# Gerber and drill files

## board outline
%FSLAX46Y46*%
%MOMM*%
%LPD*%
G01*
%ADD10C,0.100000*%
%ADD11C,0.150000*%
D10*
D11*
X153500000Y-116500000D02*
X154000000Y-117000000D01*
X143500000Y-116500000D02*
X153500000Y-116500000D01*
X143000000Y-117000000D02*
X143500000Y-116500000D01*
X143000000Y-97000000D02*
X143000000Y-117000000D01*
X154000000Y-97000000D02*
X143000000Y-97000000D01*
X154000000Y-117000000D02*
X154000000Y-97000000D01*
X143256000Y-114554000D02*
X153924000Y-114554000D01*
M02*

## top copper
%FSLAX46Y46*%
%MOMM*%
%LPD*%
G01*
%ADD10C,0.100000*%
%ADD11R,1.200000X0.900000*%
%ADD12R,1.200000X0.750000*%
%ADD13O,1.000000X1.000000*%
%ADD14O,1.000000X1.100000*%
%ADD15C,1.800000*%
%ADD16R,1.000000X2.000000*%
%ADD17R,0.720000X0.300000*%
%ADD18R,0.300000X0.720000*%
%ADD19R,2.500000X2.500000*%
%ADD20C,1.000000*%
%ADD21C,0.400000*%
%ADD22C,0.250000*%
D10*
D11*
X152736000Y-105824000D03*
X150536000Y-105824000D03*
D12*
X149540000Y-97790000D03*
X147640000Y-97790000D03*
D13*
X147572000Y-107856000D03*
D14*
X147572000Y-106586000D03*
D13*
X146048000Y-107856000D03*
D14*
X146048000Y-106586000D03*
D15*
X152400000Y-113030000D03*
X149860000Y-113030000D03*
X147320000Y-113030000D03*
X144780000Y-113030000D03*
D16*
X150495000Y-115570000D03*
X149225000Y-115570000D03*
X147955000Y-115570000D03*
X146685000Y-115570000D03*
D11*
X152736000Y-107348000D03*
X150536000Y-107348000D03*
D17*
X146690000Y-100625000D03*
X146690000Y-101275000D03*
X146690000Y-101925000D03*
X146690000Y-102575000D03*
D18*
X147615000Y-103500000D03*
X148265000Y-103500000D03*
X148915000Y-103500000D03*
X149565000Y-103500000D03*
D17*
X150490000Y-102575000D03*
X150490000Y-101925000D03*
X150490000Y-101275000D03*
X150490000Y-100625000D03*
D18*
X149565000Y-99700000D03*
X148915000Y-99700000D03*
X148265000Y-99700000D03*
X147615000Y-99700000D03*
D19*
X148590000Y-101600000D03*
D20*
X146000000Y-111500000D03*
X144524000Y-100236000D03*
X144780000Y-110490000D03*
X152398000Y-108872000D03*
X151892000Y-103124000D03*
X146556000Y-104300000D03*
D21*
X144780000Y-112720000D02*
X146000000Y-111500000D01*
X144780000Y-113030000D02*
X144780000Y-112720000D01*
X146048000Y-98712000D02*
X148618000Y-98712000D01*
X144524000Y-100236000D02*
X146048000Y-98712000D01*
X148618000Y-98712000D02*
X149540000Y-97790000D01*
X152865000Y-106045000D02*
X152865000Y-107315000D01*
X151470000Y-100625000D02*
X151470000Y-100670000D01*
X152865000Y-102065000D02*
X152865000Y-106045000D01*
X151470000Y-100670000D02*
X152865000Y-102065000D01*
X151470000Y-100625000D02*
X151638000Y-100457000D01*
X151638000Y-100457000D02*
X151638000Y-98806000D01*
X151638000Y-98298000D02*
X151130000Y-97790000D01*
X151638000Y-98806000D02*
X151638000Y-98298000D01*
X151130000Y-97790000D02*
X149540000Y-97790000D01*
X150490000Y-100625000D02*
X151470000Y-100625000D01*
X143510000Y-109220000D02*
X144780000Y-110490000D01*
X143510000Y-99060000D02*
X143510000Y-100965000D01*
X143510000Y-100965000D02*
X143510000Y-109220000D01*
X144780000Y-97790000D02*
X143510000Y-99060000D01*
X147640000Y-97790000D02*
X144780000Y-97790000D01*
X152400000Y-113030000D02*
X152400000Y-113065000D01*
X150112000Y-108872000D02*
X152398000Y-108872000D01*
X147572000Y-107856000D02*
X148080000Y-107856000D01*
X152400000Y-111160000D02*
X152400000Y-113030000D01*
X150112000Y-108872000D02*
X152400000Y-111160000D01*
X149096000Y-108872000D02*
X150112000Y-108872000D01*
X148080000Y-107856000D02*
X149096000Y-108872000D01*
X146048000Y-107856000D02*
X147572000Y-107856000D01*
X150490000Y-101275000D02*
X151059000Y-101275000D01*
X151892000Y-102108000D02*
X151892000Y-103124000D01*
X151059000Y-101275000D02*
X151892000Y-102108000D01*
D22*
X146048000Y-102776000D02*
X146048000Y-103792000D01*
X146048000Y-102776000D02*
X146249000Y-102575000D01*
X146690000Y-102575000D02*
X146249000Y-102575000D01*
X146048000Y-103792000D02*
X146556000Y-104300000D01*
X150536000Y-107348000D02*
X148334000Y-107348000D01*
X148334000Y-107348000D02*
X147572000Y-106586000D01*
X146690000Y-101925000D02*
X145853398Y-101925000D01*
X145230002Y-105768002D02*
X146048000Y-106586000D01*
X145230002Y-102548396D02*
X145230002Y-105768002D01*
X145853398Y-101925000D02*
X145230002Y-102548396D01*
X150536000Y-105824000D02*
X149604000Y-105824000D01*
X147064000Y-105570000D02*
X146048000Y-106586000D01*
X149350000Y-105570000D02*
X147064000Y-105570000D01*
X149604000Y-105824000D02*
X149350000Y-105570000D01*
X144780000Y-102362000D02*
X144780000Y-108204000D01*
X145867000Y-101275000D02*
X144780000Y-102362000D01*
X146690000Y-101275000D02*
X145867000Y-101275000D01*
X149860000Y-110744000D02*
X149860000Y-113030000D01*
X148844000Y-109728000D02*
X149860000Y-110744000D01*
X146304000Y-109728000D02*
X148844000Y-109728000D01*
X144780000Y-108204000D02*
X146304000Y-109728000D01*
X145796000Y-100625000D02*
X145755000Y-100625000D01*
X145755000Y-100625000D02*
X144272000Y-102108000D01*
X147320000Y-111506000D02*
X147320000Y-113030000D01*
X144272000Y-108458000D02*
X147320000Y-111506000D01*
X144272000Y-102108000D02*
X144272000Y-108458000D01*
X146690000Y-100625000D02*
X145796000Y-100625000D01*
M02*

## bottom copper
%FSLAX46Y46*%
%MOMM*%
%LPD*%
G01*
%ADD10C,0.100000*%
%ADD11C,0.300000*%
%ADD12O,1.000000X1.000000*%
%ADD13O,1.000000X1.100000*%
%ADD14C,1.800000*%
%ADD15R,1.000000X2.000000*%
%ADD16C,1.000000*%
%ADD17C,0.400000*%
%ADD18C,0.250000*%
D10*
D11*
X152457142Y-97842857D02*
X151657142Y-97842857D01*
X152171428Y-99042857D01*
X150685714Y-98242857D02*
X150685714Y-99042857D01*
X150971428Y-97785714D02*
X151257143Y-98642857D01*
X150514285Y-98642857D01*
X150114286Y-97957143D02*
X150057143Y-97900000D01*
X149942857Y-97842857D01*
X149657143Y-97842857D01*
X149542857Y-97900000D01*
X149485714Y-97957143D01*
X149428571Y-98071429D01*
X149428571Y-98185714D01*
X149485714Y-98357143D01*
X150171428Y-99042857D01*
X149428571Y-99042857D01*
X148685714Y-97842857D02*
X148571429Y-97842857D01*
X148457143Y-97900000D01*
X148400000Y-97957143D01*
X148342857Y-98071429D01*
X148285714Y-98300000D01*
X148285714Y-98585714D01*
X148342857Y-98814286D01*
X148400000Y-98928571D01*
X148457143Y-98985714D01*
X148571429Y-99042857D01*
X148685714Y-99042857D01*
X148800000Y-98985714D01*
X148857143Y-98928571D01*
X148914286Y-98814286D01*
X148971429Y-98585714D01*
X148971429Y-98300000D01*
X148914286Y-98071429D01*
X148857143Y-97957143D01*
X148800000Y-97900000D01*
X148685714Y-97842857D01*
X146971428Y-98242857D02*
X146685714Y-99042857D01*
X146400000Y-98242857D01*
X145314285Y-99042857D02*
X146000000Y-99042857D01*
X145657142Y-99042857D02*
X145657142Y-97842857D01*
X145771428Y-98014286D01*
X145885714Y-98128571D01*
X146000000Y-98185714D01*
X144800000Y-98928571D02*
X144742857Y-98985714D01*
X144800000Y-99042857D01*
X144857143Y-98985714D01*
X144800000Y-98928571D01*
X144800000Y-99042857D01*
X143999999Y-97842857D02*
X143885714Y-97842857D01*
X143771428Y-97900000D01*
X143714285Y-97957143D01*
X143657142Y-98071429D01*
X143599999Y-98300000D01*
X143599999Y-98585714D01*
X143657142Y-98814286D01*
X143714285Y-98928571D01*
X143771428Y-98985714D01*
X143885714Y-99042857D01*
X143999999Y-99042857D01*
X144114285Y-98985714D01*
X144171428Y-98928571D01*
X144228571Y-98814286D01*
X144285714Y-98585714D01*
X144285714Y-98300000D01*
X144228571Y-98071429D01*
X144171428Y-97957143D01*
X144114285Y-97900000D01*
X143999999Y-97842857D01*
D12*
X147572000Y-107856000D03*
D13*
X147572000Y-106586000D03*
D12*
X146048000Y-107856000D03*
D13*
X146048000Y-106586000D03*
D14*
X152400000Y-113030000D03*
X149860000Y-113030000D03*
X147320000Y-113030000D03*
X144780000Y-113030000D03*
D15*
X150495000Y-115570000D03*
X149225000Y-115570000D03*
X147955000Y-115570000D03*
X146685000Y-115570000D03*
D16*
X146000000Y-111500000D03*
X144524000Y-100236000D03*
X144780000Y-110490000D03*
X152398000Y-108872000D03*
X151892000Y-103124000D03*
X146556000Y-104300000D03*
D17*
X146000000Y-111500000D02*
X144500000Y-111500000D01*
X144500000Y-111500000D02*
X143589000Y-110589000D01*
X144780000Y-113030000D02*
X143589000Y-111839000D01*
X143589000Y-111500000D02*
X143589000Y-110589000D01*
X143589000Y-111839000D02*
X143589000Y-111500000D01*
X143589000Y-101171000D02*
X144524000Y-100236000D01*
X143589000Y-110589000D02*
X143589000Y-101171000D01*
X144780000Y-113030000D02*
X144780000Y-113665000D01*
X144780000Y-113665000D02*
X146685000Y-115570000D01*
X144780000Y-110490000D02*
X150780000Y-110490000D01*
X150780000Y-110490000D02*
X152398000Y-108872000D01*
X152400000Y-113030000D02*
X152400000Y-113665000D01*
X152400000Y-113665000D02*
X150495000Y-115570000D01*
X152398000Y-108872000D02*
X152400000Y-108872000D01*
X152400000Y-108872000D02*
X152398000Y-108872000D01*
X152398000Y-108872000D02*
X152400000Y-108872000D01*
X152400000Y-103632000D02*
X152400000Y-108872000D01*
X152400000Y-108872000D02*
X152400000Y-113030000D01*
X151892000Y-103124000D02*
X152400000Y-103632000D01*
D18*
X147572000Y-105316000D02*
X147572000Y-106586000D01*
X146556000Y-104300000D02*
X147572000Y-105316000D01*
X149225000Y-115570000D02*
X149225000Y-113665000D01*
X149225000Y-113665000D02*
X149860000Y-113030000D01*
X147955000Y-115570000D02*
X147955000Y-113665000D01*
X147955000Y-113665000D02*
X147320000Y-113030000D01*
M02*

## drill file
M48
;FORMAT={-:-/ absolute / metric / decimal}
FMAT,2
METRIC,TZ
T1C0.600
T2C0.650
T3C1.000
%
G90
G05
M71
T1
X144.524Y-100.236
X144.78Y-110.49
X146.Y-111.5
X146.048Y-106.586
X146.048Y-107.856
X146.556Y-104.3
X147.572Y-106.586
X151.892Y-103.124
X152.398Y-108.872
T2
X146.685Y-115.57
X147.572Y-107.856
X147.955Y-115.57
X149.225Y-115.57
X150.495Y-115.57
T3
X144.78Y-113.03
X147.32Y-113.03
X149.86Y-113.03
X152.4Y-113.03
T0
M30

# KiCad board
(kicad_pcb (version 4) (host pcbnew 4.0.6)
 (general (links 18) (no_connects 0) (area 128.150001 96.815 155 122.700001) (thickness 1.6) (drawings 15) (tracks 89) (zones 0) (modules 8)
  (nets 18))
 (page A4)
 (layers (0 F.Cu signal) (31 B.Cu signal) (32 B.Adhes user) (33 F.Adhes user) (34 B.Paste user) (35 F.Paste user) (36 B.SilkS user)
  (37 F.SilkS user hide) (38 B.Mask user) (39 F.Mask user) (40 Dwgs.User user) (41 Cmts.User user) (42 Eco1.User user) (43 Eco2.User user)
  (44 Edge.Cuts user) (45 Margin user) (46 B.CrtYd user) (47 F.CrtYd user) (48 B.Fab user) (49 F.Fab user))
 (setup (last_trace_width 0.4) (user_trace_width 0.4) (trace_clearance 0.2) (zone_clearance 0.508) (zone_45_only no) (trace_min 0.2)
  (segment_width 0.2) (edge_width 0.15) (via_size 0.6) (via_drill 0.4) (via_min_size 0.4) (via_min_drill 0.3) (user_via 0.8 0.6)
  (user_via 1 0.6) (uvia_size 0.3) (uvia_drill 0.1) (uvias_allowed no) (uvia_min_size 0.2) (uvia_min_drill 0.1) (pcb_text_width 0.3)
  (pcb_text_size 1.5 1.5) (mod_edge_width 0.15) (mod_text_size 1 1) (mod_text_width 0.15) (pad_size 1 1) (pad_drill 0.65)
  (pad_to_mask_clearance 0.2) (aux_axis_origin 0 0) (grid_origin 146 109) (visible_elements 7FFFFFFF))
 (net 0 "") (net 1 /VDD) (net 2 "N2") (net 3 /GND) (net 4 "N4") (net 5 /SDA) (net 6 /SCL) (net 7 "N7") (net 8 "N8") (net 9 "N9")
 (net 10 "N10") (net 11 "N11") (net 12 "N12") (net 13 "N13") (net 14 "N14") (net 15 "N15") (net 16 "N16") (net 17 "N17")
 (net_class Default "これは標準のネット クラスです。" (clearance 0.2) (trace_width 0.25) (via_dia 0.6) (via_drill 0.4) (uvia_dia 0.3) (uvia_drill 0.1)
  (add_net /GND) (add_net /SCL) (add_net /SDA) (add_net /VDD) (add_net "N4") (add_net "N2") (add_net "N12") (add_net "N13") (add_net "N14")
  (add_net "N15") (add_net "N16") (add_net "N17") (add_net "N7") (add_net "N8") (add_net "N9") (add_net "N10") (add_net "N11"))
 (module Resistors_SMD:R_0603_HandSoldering (layer F.Cu) (at 151.636 105.824 180)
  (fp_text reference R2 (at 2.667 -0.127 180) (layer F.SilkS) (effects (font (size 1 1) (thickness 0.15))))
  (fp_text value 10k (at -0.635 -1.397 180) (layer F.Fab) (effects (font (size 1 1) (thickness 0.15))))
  (pad 1 smd rect (at -1.1 0 180) (size 1.2 0.9) (layers F.Cu F.Paste F.Mask) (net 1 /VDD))
  (pad 2 smd rect (at 1.1 0 180) (size 1.2 0.9) (layers F.Cu F.Paste F.Mask) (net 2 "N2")))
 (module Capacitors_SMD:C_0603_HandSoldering (layer F.Cu) (at 148.59 97.79 180)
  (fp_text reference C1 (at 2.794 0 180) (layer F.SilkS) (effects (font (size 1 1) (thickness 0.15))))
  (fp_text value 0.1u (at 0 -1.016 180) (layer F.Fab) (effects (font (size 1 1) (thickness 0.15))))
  (pad 1 smd rect (at -0.95 0 180) (size 1.2 0.75) (layers F.Cu F.Paste F.Mask) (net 1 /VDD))
  (pad 2 smd rect (at 0.95 0 180) (size 1.2 0.75) (layers F.Cu F.Paste F.Mask) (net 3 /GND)))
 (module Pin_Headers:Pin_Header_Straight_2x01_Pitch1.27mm (layer F.Cu) (at 147.572 107.856 90)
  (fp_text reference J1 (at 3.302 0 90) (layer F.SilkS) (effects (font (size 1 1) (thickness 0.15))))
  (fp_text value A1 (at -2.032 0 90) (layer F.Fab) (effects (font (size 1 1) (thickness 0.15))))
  (pad 1 thru_hole oval (at 0 0 90) (size 1 1) (drill 0.65) (layers *.Cu *.Mask) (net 3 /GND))
  (pad 2 thru_hole oval (at 1.27 0 90) (size 1.1 1) (drill 0.6) (layers *.Cu *.Mask) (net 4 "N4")))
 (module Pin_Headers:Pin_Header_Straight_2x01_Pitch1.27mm (layer F.Cu) (at 146.048 107.856 90)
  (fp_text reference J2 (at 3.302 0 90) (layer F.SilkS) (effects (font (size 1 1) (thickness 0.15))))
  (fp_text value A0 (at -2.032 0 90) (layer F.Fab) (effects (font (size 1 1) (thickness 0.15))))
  (pad 1 thru_hole oval (at 0 0 90) (size 1 1) (drill 0.6) (layers *.Cu *.Mask) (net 3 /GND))
  (pad 2 thru_hole oval (at 1.27 0 90) (size 1.1 1) (drill 0.6) (layers *.Cu *.Mask) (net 2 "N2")))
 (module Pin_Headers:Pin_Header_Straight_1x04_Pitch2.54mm (layer F.Cu) (at 152.4 113.03 270)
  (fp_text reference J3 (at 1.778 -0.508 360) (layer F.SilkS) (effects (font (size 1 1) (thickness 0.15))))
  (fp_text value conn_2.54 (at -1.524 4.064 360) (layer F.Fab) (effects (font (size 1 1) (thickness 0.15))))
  (pad 1 thru_hole circle (at 0 0 270) (size 1.8 1.8) (drill 1) (layers *.Cu *.Mask) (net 3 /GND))
  (pad 2 thru_hole circle (at 0 2.54 270) (size 1.8 1.8) (drill 1) (layers *.Cu *.Mask) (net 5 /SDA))
  (pad 3 thru_hole circle (at 0 5.08 270) (size 1.8 1.8) (drill 1) (layers *.Cu *.Mask) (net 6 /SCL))
  (pad 4 thru_hole circle (at 0 7.62 270) (size 1.8 1.8) (drill 1) (layers *.Cu *.Mask) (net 1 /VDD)))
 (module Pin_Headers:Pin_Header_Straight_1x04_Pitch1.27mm (layer F.Cu) (at 150.495 115.57 270)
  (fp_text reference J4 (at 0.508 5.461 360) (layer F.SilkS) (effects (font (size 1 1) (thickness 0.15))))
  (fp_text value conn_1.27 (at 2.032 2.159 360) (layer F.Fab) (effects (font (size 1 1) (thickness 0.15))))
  (pad 1 thru_hole rect (at 0 0 270) (size 2 1) (drill 0.65) (layers *.Cu *.Mask) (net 3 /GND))
  (pad 2 thru_hole rect (at 0 1.27 270) (size 2 1) (drill 0.65) (layers *.Cu *.Mask) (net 5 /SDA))
  (pad 3 thru_hole rect (at 0 2.54 270) (size 2 1) (drill 0.65) (layers *.Cu *.Mask) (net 6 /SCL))
  (pad 4 thru_hole rect (at 0 3.81 270) (size 2 1) (drill 0.65) (layers *.Cu *.Mask) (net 1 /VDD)))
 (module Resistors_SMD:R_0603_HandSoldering (layer F.Cu) (at 151.636 107.348 180)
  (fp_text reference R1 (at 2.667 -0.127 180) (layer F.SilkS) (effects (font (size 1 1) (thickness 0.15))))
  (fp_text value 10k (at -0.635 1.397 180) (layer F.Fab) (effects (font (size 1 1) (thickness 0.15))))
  (pad 1 smd rect (at -1.1 0 180) (size 1.2 0.9) (layers F.Cu F.Paste F.Mask) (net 1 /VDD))
  (pad 2 smd rect (at 1.1 0 180) (size 1.2 0.9) (layers F.Cu F.Paste F.Mask) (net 4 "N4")))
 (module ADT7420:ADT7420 (layer F.Cu) (at 148.59 101.6) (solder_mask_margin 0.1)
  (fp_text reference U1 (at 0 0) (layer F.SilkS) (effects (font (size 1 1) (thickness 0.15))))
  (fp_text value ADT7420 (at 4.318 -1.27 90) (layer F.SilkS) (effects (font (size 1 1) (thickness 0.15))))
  (pad 1 smd rect (at -1.9 -0.975 90) (size 0.3 0.72) (layers F.Cu F.Paste F.Mask) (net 6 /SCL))
  (pad 2 smd rect (at -1.9 -0.325 90) (size 0.3 0.72) (layers F.Cu F.Paste F.Mask) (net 5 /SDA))
  (pad 3 smd rect (at -1.9 0.325 90) (size 0.3 0.72) (layers F.Cu F.Paste F.Mask) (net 2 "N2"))
  (pad 4 smd rect (at -1.9 0.975 90) (size 0.3 0.72) (layers F.Cu F.Paste F.Mask) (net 4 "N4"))
  (pad 5 smd rect (at -0.975 1.9) (size 0.3 0.72) (layers F.Cu F.Paste F.Mask) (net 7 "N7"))
  (pad 6 smd rect (at -0.325 1.9) (size 0.3 0.72) (layers F.Cu F.Paste F.Mask) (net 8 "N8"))
  (pad 7 smd rect (at 0.325 1.9) (size 0.3 0.72) (layers F.Cu F.Paste F.Mask) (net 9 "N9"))
  (pad 8 smd rect (at 0.975 1.9) (size 0.3 0.72) (layers F.Cu F.Paste F.Mask) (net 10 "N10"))
  (pad 9 smd rect (at 1.9 0.975 90) (size 0.3 0.72) (layers F.Cu F.Paste F.Mask) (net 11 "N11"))
  (pad 10 smd rect (at 1.9 0.325 90) (size 0.3 0.72) (layers F.Cu F.Paste F.Mask) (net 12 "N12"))
  (pad 11 smd rect (at 1.9 -0.325 90) (size 0.3 0.72) (layers F.Cu F.Paste F.Mask) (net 3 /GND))
  (pad 12 smd rect (at 1.9 -0.975 90) (size 0.3 0.72) (layers F.Cu F.Paste F.Mask) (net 1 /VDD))
  (pad 13 smd rect (at 0.975 -1.9) (size 0.3 0.72) (layers F.Cu F.Paste F.Mask) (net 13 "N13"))
  (pad 14 smd rect (at 0.325 -1.9) (size 0.3 0.72) (layers F.Cu F.Paste F.Mask) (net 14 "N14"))
  (pad 15 smd rect (at -0.325 -1.9) (size 0.3 0.72) (layers F.Cu F.Paste F.Mask) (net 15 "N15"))
  (pad 16 smd rect (at -0.975 -1.9) (size 0.3 0.72) (layers F.Cu F.Paste F.Mask) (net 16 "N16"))
  (pad 17 smd rect (at 0 0) (size 2.5 2.5) (layers F.Cu F.Paste F.Mask) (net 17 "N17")))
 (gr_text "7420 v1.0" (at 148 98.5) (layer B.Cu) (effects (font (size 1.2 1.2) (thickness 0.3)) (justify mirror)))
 (gr_line (start 153.5 116.5) (end 154 117) (angle 90) (layer Edge.Cuts) (width 0.15))
 (gr_line (start 143.5 116.5) (end 153.5 116.5) (angle 90) (layer Edge.Cuts) (width 0.15))
 (gr_line (start 143 117) (end 143.5 116.5) (angle 90) (layer Edge.Cuts) (width 0.15))
 (gr_line (start 143 97) (end 143 117) (angle 90) (layer Edge.Cuts) (width 0.15))
 (gr_line (start 154 97) (end 143 97) (angle 90) (layer Edge.Cuts) (width 0.15))
 (gr_line (start 154 117) (end 154 97) (angle 90) (layer Edge.Cuts) (width 0.15))
 (gr_line (start 143.256 114.554) (end 153.924 114.554) (angle 90) (layer Edge.Cuts) (width 0.15))
 (segment (start 146 111.5) (end 144.5 111.5) (width 0.4) (layer B.Cu) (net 1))
 (via (at 146 111.5) (size 1) (drill 0.6) (layers F.Cu B.Cu) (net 1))
 (segment (start 144.78 112.72) (end 146 111.5) (width 0.4) (layer F.Cu) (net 1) (status 400000))
 (segment (start 144.5 111.5) (end 143.589 110.589) (width 0.4) (layer B.Cu) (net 1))
 (segment (start 144.78 113.03) (end 144.78 112.72) (width 0.4) (layer F.Cu) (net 1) (status C00000))
 (segment (start 144.78 113.03) (end 143.589 111.839) (width 0.4) (layer B.Cu) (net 1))
 (segment (start 143.589 111.5) (end 143.589 110.589) (width 0.4) (layer B.Cu) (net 1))
 (segment (start 143.589 111.839) (end 143.589 111.5) (width 0.4) (layer B.Cu) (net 1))
 (segment (start 146.048 98.712) (end 148.618 98.712) (width 0.4) (layer F.Cu) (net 1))
 (segment (start 144.524 100.236) (end 146.048 98.712) (width 0.4) (layer F.Cu) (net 1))
 (segment (start 143.589 101.171) (end 144.524 100.236) (width 0.4) (layer B.Cu) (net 1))
 (via (at 144.524 100.236) (size 1) (drill 0.6) (layers F.Cu B.Cu) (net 1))
 (segment (start 143.589 110.589) (end 143.589 101.171) (width 0.4) (layer B.Cu) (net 1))
 (segment (start 148.618 98.712) (end 149.54 97.79) (width 0.4) (layer F.Cu) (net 1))
 (segment (start 144.78 113.03) (end 144.78 113.665) (width 0.4) (layer B.Cu) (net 1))
 (segment (start 144.78 113.665) (end 146.685 115.57) (width 0.4) (layer B.Cu) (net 1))
 (segment (start 152.865 106.045) (end 152.865 107.315) (width 0.4) (layer F.Cu) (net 1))
 (segment (start 151.47 100.625) (end 151.47 100.67) (width 0.4) (layer F.Cu) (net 1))
 (segment (start 152.865 102.065) (end 152.865 106.045) (width 0.4) (layer F.Cu) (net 1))
 (segment (start 151.47 100.67) (end 152.865 102.065) (width 0.4) (layer F.Cu) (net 1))
 (segment (start 151.47 100.625) (end 151.638 100.457) (width 0.4) (layer F.Cu) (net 1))
 (segment (start 151.638 100.457) (end 151.638 98.806) (width 0.4) (layer F.Cu) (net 1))
 (segment (start 151.638 98.298) (end 151.13 97.79) (width 0.4) (layer F.Cu) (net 1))
 (segment (start 151.638 98.806) (end 151.638 98.298) (width 0.4) (layer F.Cu) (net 1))
 (segment (start 151.13 97.79) (end 149.54 97.79) (width 0.4) (layer F.Cu) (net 1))
 (segment (start 150.49 100.625) (end 151.47 100.625) (width 0.4) (layer F.Cu) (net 1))
 (segment (start 144.78 110.49) (end 150.78 110.49) (width 0.4) (layer B.Cu) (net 3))
 (via (at 144.78 110.49) (size 1) (drill 0.6) (layers F.Cu B.Cu) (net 3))
 (segment (start 143.51 109.22) (end 144.78 110.49) (width 0.4) (layer F.Cu) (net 3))
 (segment (start 143.51 99.06) (end 143.51 100.965) (width 0.4) (layer F.Cu) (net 3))
 (segment (start 143.51 100.965) (end 143.51 109.22) (width 0.4) (layer F.Cu) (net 3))
 (segment (start 144.78 97.79) (end 143.51 99.06) (width 0.4) (layer F.Cu) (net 3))
 (segment (start 147.64 97.79) (end 144.78 97.79) (width 0.4) (layer F.Cu) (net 3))
 (segment (start 150.78 110.49) (end 152.398 108.872) (width 0.4) (layer B.Cu) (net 3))
 (segment (start 152.4 113.03) (end 152.4 113.665) (width 0.4) (layer B.Cu) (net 3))
 (segment (start 152.4 113.665) (end 150.495 115.57) (width 0.4) (layer B.Cu) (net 3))
 (segment (start 152.4 113.03) (end 152.4 113.065) (width 0.4) (layer F.Cu) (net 3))
 (segment (start 150.112 108.872) (end 152.398 108.872) (width 0.4) (layer F.Cu) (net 3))
 (via (at 152.398 108.872) (size 1) (drill 0.6) (layers F.Cu B.Cu) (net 3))
 (segment (start 152.398 108.872) (end 152.4 108.872) (width 0.4) (layer B.Cu) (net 3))
 (segment (start 152.4 108.872) (end 152.398 108.872) (width 0.4) (layer B.Cu) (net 3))
 (segment (start 152.398 108.872) (end 152.4 108.872) (width 0.4) (layer B.Cu) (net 3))
 (segment (start 147.572 107.856) (end 148.08 107.856) (width 0.4) (layer F.Cu) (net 3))
 (segment (start 152.4 111.16) (end 152.4 113.03) (width 0.4) (layer F.Cu) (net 3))
 (segment (start 150.112 108.872) (end 152.4 111.16) (width 0.4) (layer F.Cu) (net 3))
 (segment (start 149.096 108.872) (end 150.112 108.872) (width 0.4) (layer F.Cu) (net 3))
 (segment (start 148.08 107.856) (end 149.096 108.872) (width 0.4) (layer F.Cu) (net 3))
 (segment (start 146.048 107.856) (end 147.572 107.856) (width 0.4) (layer F.Cu) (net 3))
 (segment (start 150.49 101.275) (end 151.059 101.275) (width 0.4) (layer F.Cu) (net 3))
 (segment (start 152.4 103.632) (end 152.4 108.872) (width 0.4) (layer B.Cu) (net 3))
 (segment (start 152.4 108.872) (end 152.4 113.03) (width 0.4) (layer B.Cu) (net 3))
 (segment (start 151.892 103.124) (end 152.4 103.632) (width 0.4) (layer B.Cu) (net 3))
 (via (at 151.892 103.124) (size 1) (drill 0.6) (layers F.Cu B.Cu) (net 3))
 (segment (start 151.892 102.108) (end 151.892 103.124) (width 0.4) (layer F.Cu) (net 3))
 (segment (start 151.059 101.275) (end 151.892 102.108) (width 0.4) (layer F.Cu) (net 3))
 (segment (start 146.048 102.776) (end 146.048 103.792) (width 0.25) (layer F.Cu) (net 4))
 (segment (start 146.048 102.776) (end 146.249 102.575) (width 0.25) (layer F.Cu) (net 4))
 (segment (start 146.69 102.575) (end 146.249 102.575) (width 0.25) (layer F.Cu) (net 4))
 (segment (start 147.572 105.316) (end 147.572 106.586) (width 0.25) (layer B.Cu) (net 4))
 (segment (start 146.556 104.3) (end 147.572 105.316) (width 0.25) (layer B.Cu) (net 4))
 (via (at 146.556 104.3) (size 1) (drill 0.6) (layers F.Cu B.Cu) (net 4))
 (segment (start 146.048 103.792) (end 146.556 104.3) (width 0.25) (layer F.Cu) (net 4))
 (segment (start 150.536 107.348) (end 148.334 107.348) (width 0.25) (layer F.Cu) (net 4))
 (segment (start 148.334 107.348) (end 147.572 106.586) (width 0.25) (layer F.Cu) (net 4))
 (segment (start 146.69 101.925) (end 145.853398 101.925) (width 0.25) (layer F.Cu) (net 2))
 (segment (start 145.230002 105.768002) (end 146.048 106.586) (width 0.25) (layer F.Cu) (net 2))
 (segment (start 145.230002 102.548396) (end 145.230002 105.768002) (width 0.25) (layer F.Cu) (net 2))
 (segment (start 145.853398 101.925) (end 145.230002 102.548396) (width 0.25) (layer F.Cu) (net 2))
 (segment (start 150.536 105.824) (end 149.604 105.824) (width 0.25) (layer F.Cu) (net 2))
 (segment (start 147.064 105.57) (end 146.048 106.586) (width 0.25) (layer F.Cu) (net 2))
 (segment (start 149.35 105.57) (end 147.064 105.57) (width 0.25) (layer F.Cu) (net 2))
 (segment (start 149.604 105.824) (end 149.35 105.57) (width 0.25) (layer F.Cu) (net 2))
 (segment (start 144.78 102.362) (end 144.78 108.204) (width 0.25) (layer F.Cu) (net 5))
 (segment (start 145.867 101.275) (end 144.78 102.362) (width 0.25) (layer F.Cu) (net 5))
 (segment (start 146.69 101.275) (end 145.867 101.275) (width 0.25) (layer F.Cu) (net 5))
 (segment (start 149.86 110.744) (end 149.86 113.03) (width 0.25) (layer F.Cu) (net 5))
 (segment (start 148.844 109.728) (end 149.86 110.744) (width 0.25) (layer F.Cu) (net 5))
 (segment (start 146.304 109.728) (end 148.844 109.728) (width 0.25) (layer F.Cu) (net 5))
 (segment (start 144.78 108.204) (end 146.304 109.728) (width 0.25) (layer F.Cu) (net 5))
 (segment (start 149.225 115.57) (end 149.225 113.665) (width 0.25) (layer B.Cu) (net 5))
 (segment (start 149.225 113.665) (end 149.86 113.03) (width 0.25) (layer B.Cu) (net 5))
 (segment (start 145.796 100.625) (end 145.755 100.625) (width 0.25) (layer F.Cu) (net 6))
 (segment (start 145.755 100.625) (end 144.272 102.108) (width 0.25) (layer F.Cu) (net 6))
 (segment (start 147.32 111.506) (end 147.32 113.03) (width 0.25) (layer F.Cu) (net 6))
 (segment (start 144.272 108.458) (end 147.32 111.506) (width 0.25) (layer F.Cu) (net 6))
 (segment (start 144.272 102.108) (end 144.272 108.458) (width 0.25) (layer F.Cu) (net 6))
 (segment (start 147.955 115.57) (end 147.955 113.665) (width 0.25) (layer B.Cu) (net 6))
 (segment (start 147.955 113.665) (end 147.32 113.03) (width 0.25) (layer B.Cu) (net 6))
 (segment (start 146.69 100.625) (end 145.796 100.625) (width 0.25) (layer F.Cu) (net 6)))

